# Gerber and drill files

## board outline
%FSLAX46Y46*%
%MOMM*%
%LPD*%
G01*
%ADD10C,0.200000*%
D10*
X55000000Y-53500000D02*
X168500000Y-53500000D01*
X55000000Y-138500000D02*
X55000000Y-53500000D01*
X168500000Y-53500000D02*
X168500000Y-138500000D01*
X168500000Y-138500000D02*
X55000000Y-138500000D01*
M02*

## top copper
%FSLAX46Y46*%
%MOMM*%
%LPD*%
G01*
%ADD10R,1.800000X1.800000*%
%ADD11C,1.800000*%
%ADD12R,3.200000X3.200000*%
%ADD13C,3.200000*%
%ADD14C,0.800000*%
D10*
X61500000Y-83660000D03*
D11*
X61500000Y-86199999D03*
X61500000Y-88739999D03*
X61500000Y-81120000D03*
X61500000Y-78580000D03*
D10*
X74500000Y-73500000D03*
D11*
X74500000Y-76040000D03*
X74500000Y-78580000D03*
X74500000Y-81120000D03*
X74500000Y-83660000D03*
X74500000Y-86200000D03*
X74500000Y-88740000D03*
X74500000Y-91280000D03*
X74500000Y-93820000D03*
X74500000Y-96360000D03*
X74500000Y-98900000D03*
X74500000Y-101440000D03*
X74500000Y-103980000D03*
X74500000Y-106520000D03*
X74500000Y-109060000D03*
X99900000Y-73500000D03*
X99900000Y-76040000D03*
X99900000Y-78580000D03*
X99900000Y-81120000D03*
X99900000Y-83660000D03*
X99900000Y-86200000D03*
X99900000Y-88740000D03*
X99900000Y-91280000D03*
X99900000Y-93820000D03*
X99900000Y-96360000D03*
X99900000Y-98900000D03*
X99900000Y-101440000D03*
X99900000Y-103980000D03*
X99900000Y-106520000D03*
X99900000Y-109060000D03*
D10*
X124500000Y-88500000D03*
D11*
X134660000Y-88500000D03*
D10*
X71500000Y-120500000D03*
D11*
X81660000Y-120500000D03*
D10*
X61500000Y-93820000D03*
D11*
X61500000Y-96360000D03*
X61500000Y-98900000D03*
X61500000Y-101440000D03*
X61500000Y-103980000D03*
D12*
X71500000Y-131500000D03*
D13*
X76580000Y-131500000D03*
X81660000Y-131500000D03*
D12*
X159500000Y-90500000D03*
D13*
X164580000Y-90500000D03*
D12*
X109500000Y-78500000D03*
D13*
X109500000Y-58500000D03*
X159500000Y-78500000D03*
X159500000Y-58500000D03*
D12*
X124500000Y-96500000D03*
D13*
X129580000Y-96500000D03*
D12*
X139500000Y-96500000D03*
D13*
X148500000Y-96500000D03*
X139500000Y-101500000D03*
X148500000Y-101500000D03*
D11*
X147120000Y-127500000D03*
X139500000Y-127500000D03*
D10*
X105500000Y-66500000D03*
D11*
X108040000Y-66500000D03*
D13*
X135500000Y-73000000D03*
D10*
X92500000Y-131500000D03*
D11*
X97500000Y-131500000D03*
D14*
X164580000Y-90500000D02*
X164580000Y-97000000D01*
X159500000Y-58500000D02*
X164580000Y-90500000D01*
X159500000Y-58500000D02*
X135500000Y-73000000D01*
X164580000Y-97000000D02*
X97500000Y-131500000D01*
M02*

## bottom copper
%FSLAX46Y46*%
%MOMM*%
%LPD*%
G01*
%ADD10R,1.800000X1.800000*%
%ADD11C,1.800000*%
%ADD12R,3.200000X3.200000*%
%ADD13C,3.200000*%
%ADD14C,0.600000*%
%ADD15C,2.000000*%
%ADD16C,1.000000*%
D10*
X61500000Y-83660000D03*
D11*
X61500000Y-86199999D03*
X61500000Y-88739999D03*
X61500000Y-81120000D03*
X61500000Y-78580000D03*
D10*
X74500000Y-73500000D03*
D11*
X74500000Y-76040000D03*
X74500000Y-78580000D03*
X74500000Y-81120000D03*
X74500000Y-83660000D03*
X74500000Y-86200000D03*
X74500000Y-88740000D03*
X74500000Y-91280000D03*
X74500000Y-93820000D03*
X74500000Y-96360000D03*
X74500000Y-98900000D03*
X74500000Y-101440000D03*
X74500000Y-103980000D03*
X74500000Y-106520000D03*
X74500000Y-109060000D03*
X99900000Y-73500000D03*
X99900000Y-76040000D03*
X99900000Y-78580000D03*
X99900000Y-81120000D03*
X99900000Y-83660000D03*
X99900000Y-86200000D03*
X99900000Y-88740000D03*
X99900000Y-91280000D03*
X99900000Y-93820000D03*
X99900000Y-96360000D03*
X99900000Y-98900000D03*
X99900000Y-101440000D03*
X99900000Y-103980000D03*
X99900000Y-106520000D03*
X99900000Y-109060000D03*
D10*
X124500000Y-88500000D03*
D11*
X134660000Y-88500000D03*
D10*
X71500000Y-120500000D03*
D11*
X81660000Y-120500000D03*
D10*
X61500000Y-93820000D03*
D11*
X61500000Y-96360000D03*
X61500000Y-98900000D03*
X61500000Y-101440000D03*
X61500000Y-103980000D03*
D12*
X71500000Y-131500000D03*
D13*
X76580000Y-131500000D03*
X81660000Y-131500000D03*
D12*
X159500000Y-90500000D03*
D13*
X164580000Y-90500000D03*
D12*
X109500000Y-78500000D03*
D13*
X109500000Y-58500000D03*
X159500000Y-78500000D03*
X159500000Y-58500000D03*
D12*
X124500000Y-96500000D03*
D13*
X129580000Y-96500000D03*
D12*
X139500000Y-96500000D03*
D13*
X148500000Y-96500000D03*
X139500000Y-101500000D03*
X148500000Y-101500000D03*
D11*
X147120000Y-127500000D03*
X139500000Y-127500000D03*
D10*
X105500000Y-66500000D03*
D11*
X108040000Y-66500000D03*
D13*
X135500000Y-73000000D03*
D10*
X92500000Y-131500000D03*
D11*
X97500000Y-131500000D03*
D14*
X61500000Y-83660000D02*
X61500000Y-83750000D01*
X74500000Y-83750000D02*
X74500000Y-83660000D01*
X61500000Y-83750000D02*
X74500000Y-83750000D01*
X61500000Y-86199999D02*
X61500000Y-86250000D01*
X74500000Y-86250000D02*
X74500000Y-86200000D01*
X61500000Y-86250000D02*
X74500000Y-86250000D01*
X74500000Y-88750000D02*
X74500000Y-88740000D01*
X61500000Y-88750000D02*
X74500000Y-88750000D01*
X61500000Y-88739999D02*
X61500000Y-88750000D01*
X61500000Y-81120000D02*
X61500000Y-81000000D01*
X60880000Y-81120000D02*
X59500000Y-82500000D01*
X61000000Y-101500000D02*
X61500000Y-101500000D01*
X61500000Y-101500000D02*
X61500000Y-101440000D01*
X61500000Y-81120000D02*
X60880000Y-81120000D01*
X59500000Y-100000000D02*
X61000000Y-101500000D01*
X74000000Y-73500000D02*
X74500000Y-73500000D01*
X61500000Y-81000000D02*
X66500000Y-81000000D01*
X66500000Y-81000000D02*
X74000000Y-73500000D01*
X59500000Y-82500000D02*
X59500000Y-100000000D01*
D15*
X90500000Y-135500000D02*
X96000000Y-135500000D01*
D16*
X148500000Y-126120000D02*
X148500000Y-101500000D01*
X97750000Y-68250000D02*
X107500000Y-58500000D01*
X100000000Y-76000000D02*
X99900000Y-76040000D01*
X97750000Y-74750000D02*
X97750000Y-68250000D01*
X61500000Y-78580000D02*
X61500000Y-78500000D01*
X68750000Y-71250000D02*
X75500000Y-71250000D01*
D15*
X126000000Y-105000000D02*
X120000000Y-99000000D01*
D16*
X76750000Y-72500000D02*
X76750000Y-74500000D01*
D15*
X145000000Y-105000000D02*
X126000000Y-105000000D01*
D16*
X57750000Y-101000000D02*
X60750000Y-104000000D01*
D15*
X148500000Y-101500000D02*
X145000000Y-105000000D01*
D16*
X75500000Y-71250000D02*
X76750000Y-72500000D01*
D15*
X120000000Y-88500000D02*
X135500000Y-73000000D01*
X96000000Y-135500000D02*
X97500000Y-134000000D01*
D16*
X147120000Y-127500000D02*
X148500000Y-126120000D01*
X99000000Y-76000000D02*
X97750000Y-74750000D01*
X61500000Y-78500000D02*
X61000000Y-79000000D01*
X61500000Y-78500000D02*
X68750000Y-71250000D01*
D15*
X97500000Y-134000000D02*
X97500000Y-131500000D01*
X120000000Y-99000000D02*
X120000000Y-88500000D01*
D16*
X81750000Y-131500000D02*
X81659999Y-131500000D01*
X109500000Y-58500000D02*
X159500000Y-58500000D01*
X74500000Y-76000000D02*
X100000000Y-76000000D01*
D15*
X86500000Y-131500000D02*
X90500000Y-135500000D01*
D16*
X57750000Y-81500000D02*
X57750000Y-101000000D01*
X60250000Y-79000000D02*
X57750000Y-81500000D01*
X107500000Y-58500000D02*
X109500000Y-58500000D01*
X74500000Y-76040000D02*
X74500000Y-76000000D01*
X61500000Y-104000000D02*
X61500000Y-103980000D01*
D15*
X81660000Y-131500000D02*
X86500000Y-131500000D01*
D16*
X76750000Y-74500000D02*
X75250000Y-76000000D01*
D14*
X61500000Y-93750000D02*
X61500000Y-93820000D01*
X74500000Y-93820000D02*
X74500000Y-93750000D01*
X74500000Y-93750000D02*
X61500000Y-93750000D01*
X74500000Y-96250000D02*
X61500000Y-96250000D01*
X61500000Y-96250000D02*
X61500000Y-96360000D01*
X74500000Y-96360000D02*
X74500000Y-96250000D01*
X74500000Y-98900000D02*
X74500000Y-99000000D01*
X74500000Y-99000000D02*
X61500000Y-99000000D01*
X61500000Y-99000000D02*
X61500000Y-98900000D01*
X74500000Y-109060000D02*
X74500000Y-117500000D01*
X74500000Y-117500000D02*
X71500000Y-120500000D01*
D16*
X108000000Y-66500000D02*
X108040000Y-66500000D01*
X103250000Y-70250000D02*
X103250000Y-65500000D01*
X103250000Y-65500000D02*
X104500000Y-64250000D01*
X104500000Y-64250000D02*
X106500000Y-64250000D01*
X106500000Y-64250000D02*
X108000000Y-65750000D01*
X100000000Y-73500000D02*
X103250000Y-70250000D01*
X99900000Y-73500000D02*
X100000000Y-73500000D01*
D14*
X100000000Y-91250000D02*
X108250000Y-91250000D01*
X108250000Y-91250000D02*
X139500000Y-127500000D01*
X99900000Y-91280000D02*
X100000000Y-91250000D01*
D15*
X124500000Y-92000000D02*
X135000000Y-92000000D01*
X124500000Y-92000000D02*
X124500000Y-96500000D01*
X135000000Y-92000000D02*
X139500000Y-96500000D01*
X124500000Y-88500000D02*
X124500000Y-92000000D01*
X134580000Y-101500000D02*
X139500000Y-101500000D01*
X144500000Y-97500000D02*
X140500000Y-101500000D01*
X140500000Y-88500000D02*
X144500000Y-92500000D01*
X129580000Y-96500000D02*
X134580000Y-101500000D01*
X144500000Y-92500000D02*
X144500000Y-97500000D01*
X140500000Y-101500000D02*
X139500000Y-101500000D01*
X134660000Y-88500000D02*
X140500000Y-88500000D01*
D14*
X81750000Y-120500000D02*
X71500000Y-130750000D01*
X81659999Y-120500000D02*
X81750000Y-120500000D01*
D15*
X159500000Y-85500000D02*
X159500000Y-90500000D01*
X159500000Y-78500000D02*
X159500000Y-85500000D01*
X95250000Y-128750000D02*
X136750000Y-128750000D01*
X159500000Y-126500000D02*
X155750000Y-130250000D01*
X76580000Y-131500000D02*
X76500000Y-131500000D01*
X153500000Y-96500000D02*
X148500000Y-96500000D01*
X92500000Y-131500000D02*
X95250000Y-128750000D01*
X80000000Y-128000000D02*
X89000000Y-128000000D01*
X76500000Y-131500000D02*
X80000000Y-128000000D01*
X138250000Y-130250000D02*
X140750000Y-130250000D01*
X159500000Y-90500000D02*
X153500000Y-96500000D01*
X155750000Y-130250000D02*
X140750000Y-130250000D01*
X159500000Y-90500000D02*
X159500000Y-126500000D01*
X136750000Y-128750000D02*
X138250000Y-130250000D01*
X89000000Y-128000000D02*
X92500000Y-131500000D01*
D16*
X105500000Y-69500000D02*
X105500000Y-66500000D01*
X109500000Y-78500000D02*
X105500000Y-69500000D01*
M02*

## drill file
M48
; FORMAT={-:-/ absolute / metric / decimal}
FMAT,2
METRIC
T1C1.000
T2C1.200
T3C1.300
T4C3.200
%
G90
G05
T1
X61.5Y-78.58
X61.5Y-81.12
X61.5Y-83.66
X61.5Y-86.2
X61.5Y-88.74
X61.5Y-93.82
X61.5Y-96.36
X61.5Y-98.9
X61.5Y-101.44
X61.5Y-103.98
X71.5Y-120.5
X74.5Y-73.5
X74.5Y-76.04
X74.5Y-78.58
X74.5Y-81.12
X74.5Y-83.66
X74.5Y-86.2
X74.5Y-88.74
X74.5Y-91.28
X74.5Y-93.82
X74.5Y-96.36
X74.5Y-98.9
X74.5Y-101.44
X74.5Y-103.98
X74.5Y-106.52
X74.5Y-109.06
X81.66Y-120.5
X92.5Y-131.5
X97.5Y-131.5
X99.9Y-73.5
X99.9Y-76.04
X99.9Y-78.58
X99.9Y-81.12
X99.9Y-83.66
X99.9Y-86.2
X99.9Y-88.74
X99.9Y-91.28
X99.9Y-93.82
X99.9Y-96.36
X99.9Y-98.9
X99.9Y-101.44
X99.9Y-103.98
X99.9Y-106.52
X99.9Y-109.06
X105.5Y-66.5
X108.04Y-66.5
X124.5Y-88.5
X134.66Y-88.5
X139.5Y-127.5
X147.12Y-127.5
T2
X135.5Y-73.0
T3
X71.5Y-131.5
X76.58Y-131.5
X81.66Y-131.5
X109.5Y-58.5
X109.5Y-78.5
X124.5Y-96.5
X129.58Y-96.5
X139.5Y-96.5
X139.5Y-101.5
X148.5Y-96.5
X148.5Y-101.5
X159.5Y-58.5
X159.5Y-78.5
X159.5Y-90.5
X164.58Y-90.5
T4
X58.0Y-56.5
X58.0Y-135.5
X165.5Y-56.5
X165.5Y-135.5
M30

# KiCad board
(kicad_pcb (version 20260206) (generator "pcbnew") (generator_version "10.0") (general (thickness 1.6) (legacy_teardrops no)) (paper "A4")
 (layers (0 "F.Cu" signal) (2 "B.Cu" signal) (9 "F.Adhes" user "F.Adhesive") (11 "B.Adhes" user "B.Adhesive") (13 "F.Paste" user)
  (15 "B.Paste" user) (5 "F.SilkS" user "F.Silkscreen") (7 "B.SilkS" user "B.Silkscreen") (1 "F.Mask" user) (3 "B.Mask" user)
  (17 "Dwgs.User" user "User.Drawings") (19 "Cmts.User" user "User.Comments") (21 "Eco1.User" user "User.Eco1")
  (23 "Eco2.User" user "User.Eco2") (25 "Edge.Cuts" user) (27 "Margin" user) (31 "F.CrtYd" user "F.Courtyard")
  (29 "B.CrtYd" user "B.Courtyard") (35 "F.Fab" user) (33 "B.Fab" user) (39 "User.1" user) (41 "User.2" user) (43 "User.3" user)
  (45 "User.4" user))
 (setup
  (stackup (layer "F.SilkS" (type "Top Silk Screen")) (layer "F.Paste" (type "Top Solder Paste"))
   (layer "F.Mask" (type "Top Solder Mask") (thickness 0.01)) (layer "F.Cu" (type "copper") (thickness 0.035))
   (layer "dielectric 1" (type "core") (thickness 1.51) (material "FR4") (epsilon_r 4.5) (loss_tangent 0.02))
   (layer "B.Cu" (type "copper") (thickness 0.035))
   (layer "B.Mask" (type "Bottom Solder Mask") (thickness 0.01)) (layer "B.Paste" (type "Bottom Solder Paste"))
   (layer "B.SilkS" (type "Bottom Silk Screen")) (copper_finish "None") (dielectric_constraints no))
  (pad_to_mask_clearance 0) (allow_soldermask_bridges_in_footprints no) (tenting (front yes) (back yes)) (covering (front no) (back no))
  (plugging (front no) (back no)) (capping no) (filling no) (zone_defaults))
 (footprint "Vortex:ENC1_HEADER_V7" (layer "F.Cu") (at 61.5 83.5 -90)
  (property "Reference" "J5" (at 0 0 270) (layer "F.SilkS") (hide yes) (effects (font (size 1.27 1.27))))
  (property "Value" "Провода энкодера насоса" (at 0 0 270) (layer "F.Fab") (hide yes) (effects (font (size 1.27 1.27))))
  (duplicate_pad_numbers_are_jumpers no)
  (pad "1" thru_hole rect (at 0.16 0 270) (size 1.8 1.8) (drill 1) (layers "*.Cu") (remove_unused_layers no) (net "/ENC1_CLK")
   (thermal_bridge_angle 45))
  (pad "2" thru_hole circle (at 2.699999 0 270) (size 1.8 1.8) (drill 1) (layers "*.Cu") (remove_unused_layers no) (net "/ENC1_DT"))
  (pad "3" thru_hole circle (at 5.239999 0 270) (size 1.8 1.8) (drill 1) (layers "*.Cu") (remove_unused_layers no) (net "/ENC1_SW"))
  (pad "4" thru_hole circle (at -2.38 0 270) (size 1.8 1.8) (drill 1) (layers "*.Cu") (remove_unused_layers no) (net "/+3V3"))
  (pad "5" thru_hole circle (at -4.92 0 270) (size 1.8 1.8) (drill 1) (layers "*.Cu") (remove_unused_layers no) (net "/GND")))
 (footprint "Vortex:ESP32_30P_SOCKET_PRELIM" (layer "F.Cu") (at 74.5 73.5)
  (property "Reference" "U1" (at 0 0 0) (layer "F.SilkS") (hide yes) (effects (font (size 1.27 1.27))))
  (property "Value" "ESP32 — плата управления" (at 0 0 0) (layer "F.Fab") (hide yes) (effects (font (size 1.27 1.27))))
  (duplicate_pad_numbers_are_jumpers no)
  (pad "1" thru_hole rect (at 0 0) (size 1.8 1.8) (drill 1) (layers "*.Cu") (remove_unused_layers no) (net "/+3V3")
   (thermal_bridge_angle 45))
  (pad "2" thru_hole circle (at 0 2.54) (size 1.8 1.8) (drill 1) (layers "*.Cu") (remove_unused_layers no) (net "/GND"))
  (pad "3" thru_hole circle (at 0 5.08) (size 1.8 1.8) (drill 1) (layers "*.Cu") (remove_unused_layers no) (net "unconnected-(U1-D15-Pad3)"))
  (pad "4" thru_hole circle (at 0 7.62) (size 1.8 1.8) (drill 1) (layers "*.Cu") (remove_unused_layers no) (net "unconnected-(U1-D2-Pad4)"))
  (pad "5" thru_hole circle (at 0 10.16) (size 1.8 1.8) (drill 1) (layers "*.Cu") (remove_unused_layers no) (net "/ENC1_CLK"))
  (pad "6" thru_hole circle (at 0 12.7) (size 1.8 1.8) (drill 1) (layers "*.Cu") (remove_unused_layers no) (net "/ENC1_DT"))
  (pad "7" thru_hole circle (at 0 15.24) (size 1.8 1.8) (drill 1) (layers "*.Cu") (remove_unused_layers no) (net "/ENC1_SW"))
  (pad "8" thru_hole circle (at 0 17.78) (size 1.8 1.8) (drill 1) (layers "*.Cu") (remove_unused_layers no) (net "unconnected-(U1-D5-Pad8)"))
  (pad "9" thru_hole circle (at 0 20.32) (size 1.8 1.8) (drill 1) (layers "*.Cu") (remove_unused_layers no) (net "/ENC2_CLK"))
  (pad "10" thru_hole circle (at 0 22.86) (size 1.8 1.8) (drill 1) (layers "*.Cu") (remove_unused_layers no) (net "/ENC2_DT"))
  (pad "11" thru_hole circle (at 0 25.4) (size 1.8 1.8) (drill 1) (layers "*.Cu") (remove_unused_layers no) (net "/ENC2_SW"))
  (pad "12" thru_hole circle (at 0 27.94) (size 1.8 1.8) (drill 1) (layers "*.Cu") (remove_unused_layers no)
   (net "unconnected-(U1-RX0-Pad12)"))
  (pad "13" thru_hole circle (at 0 30.48) (size 1.8 1.8) (drill 1) (layers "*.Cu") (remove_unused_layers no)
   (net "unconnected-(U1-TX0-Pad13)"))
  (pad "14" thru_hole circle (at 0 33.02) (size 1.8 1.8) (drill 1) (layers "*.Cu") (remove_unused_layers no)
   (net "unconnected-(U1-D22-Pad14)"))
  (pad "15" thru_hole circle (at 0 35.56) (size 1.8 1.8) (drill 1) (layers "*.Cu") (remove_unused_layers no) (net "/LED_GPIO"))
  (pad "16" thru_hole circle (at 25.4 0) (size 1.8 1.8) (drill 1) (layers "*.Cu") (remove_unused_layers no) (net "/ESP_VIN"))
  (pad "17" thru_hole circle (at 25.4 2.54) (size 1.8 1.8) (drill 1) (layers "*.Cu") (remove_unused_layers no) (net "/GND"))
  (pad "18" thru_hole circle (at 25.4 5.08) (size 1.8 1.8) (drill 1) (layers "*.Cu") (remove_unused_layers no)
   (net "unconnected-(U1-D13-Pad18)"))
  (pad "19" thru_hole circle (at 25.4 7.62) (size 1.8 1.8) (drill 1) (layers "*.Cu") (remove_unused_layers no)
   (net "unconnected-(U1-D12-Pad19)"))
  (pad "20" thru_hole circle (at 25.4 10.16) (size 1.8 1.8) (drill 1) (layers "*.Cu") (remove_unused_layers no)
   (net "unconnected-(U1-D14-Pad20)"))
  (pad "21" thru_hole circle (at 25.4 12.7) (size 1.8 1.8) (drill 1) (layers "*.Cu") (remove_unused_layers no)
   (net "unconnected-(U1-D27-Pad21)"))
  (pad "22" thru_hole circle (at 25.4 15.24) (size 1.8 1.8) (drill 1) (layers "*.Cu") (remove_unused_layers no)
   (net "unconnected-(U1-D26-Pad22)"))
  (pad "23" thru_hole circle (at 25.4 17.78) (size 1.8 1.8) (drill 1) (layers "*.Cu") (remove_unused_layers no) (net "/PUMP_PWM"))
  (pad "24" thru_hole circle (at 25.4 20.32) (size 1.8 1.8) (drill 1) (layers "*.Cu") (remove_unused_layers no)
   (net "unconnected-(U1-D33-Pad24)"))
  (pad "25" thru_hole circle (at 25.4 22.86) (size 1.8 1.8) (drill 1) (layers "*.Cu") (remove_unused_layers no)
   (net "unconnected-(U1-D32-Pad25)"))
  (pad "26" thru_hole circle (at 25.4 25.4) (size 1.8 1.8) (drill 1) (layers "*.Cu") (remove_unused_layers no)
   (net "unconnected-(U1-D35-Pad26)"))
  (pad "27" thru_hole circle (at 25.4 27.94) (size 1.8 1.8) (drill 1) (layers "*.Cu") (remove_unused_layers no)
   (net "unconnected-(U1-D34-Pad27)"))
  (pad "28" thru_hole circle (at 25.4 30.48) (size 1.8 1.8) (drill 1) (layers "*.Cu") (remove_unused_layers no)
   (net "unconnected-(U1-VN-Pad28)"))
  (pad "29" thru_hole circle (at 25.4 33.02) (size 1.8 1.8) (drill 1) (layers "*.Cu") (remove_unused_layers no)
   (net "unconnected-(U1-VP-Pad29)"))
  (pad "30" thru_hole circle (at 25.4 35.56) (size 1.8 1.8) (drill 1) (layers "*.Cu") (remove_unused_layers no)
   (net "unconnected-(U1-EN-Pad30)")))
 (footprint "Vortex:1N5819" (layer "F.Cu") (at 124.5 88.5)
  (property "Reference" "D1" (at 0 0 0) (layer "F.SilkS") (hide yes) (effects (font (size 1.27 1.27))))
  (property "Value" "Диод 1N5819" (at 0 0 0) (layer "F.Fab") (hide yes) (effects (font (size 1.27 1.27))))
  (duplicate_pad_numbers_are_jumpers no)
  (pad "1" thru_hole rect (at 0 0) (size 1.8 1.8) (drill 1) (layers "*.Cu") (remove_unused_layers no) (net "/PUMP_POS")
   (thermal_bridge_angle 45))
  (pad "2" thru_hole circle (at 10.16 0) (size 1.8 1.8) (drill 1) (layers "*.Cu") (remove_unused_layers no) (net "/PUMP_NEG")))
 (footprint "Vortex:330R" (layer "F.Cu") (at 71.5 120.5)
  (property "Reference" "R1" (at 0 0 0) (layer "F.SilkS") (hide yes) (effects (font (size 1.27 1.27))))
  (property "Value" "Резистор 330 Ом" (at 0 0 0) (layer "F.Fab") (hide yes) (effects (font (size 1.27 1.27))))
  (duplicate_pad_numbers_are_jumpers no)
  (pad "1" thru_hole rect (at 0 0) (size 1.8 1.8) (drill 1) (layers "*.Cu") (remove_unused_layers no) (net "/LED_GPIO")
   (thermal_bridge_angle 45))
  (pad "2" thru_hole circle (at 10.16 0) (size 1.8 1.8) (drill 1) (layers "*.Cu") (remove_unused_layers no) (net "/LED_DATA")))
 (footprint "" (layer "F.Cu") (at 58 135.5)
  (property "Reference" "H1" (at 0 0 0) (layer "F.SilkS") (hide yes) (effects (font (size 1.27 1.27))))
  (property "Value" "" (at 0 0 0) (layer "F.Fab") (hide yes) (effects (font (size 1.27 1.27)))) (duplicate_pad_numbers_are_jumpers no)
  (pad "" np_thru_hole circle (at 0 0) (size 3.2 3.2) (drill 3.2) (layers "*.Cu")))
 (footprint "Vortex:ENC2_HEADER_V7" (layer "F.Cu") (at 61.5 96.5 -90)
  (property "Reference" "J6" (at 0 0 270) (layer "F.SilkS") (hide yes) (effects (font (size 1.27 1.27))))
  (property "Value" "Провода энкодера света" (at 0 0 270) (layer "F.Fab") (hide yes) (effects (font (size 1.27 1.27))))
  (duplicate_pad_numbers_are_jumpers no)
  (pad "1" thru_hole rect (at -2.68 0 270) (size 1.8 1.8) (drill 1) (layers "*.Cu") (remove_unused_layers no) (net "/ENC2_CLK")
   (thermal_bridge_angle 45))
  (pad "2" thru_hole circle (at -0.14 0 270) (size 1.8 1.8) (drill 1) (layers "*.Cu") (remove_unused_layers no) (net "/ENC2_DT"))
  (pad "3" thru_hole circle (at 2.4 0 270) (size 1.8 1.8) (drill 1) (layers "*.Cu") (remove_unused_layers no) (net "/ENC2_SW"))
  (pad "4" thru_hole circle (at 4.94 0 270) (size 1.8 1.8) (drill 1) (layers "*.Cu") (remove_unused_layers no) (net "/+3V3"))
  (pad "5" thru_hole circle (at 7.48 0 270) (size 1.8 1.8) (drill 1) (layers "*.Cu") (remove_unused_layers no) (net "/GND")))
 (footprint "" (layer "F.Cu") (at 58 56.5)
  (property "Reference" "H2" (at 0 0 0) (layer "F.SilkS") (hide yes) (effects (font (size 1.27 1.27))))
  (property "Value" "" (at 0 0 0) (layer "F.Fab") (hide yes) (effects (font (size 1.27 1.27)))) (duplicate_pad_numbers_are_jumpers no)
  (pad "" np_thru_hole circle (at 0 0) (size 3.2 3.2) (drill 3.2) (layers "*.Cu")))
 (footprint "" (layer "F.Cu") (at 165.5 135.5)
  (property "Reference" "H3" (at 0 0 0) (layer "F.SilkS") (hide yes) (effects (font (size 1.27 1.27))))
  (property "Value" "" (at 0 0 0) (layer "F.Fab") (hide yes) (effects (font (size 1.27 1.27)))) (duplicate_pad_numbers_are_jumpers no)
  (pad "" np_thru_hole circle (at 0 0) (size 3.2 3.2) (drill 3.2) (layers "*.Cu")))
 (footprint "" (layer "F.Cu") (at 165.5 56.5)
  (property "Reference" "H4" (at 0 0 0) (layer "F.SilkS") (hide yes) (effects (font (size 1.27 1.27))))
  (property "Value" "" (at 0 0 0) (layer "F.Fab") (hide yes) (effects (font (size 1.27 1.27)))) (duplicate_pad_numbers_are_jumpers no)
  (pad "" np_thru_hole circle (at 0 0) (size 3.2 3.2) (drill 3.2) (layers "*.Cu")))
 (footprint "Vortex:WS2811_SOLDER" (layer "F.Cu") (at 71.5 131.5)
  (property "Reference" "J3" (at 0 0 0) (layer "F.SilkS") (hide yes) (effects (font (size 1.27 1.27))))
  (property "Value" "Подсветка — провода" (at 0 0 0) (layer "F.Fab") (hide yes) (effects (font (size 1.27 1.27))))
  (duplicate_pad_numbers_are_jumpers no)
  (pad "1" thru_hole rect (at 0 0) (size 3.2 3.2) (drill 1.3) (layers "*.Cu") (remove_unused_layers no) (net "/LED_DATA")
   (thermal_bridge_angle 45))
  (pad "2" thru_hole circle (at 5.08 0) (size 3.2 3.2) (drill 1.3) (layers "*.Cu") (remove_unused_layers no) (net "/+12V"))
  (pad "3" thru_hole circle (at 10.16 0) (size 3.2 3.2) (drill 1.3) (layers "*.Cu") (remove_unused_layers no) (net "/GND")))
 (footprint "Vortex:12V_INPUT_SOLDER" (layer "F.Cu") (at 159.5 90.5)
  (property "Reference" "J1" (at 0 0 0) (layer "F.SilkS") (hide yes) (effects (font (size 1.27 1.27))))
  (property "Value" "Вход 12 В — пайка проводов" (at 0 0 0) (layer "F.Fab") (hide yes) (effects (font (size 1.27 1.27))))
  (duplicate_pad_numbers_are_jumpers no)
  (pad "1" thru_hole rect (at 0 0) (size 3.2 3.2) (drill 1.3) (layers "*.Cu") (remove_unused_layers no) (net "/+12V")
   (thermal_bridge_angle 45))
  (pad "2" thru_hole circle (at 5.08 0) (size 3.2 3.2) (drill 1.3) (layers "*.Cu") (remove_unused_layers no) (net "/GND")))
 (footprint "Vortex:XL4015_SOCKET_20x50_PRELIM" (layer "F.Cu") (at 109.5 78.5 90)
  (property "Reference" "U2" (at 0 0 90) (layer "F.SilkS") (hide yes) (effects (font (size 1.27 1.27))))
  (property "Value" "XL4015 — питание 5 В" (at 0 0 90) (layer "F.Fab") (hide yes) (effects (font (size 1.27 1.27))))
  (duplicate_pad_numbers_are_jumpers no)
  (pad "1" thru_hole rect (at 0 0 90) (size 3.2 3.2) (drill 1.3) (layers "*.Cu") (remove_unused_layers no) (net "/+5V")
   (thermal_bridge_angle 45))
  (pad "2" thru_hole circle (at 20 0 90) (size 3.2 3.2) (drill 1.3) (layers "*.Cu") (remove_unused_layers no) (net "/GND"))
  (pad "3" thru_hole circle (at 0 50 90) (size 3.2 3.2) (drill 1.3) (layers "*.Cu") (remove_unused_layers no) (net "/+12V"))
  (pad "4" thru_hole circle (at 20 50 90) (size 3.2 3.2) (drill 1.3) (layers "*.Cu") (remove_unused_layers no) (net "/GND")))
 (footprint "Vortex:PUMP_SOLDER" (layer "F.Cu") (at 124.5 96.5)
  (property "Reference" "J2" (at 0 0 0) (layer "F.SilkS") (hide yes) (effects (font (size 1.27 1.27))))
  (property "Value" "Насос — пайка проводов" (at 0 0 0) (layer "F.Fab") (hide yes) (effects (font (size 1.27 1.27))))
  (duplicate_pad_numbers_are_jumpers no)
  (pad "1" thru_hole rect (at 0 0) (size 3.2 3.2) (drill 1.3) (layers "*.Cu") (remove_unused_layers no) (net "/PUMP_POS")
   (thermal_bridge_angle 45))
  (pad "2" thru_hole circle (at 5.08 0) (size 3.2 3.2) (drill 1.3) (layers "*.Cu") (remove_unused_layers no) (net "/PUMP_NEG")))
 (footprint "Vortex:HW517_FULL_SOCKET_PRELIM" (layer "F.Cu") (at 139.5 96.5)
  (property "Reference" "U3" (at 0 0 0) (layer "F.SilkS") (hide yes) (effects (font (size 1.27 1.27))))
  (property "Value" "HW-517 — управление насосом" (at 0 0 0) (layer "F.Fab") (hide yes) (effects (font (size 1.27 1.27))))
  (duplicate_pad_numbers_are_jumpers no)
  (pad "1" thru_hole rect (at 0 0) (size 3.2 3.2) (drill 1.3) (layers "*.Cu") (remove_unused_layers no) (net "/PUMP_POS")
   (thermal_bridge_angle 45))
  (pad "2" thru_hole circle (at 9 0) (size 3.2 3.2) (drill 1.3) (layers "*.Cu") (remove_unused_layers no) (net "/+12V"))
  (pad "3" thru_hole circle (at 0 5) (size 3.2 3.2) (drill 1.3) (layers "*.Cu") (remove_unused_layers no) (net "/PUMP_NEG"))
  (pad "4" thru_hole circle (at 9 5) (size 3.2 3.2) (drill 1.3) (layers "*.Cu") (remove_unused_layers no) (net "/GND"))
  (pad "5" thru_hole circle (at 7.62 31) (size 1.8 1.8) (drill 1) (layers "*.Cu") (remove_unused_layers no) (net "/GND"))
  (pad "6" thru_hole circle (at 0 31) (size 1.8 1.8) (drill 1) (layers "*.Cu") (remove_unused_layers no) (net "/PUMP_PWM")))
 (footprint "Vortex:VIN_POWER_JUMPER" (layer "F.Cu") (at 105.5 66.5)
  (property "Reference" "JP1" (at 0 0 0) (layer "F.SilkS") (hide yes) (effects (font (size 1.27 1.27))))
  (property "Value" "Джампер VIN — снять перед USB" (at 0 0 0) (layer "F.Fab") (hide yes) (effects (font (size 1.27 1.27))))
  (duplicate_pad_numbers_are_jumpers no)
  (pad "1" thru_hole rect (at 0 0) (size 1.8 1.8) (drill 1) (layers "*.Cu") (remove_unused_layers no) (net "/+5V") (thermal_bridge_angle 45))
  (pad "2" thru_hole circle (at 2.54 0) (size 1.8 1.8) (drill 1) (layers "*.Cu") (remove_unused_layers no) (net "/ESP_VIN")))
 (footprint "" (layer "F.Cu") (at 135.5 73)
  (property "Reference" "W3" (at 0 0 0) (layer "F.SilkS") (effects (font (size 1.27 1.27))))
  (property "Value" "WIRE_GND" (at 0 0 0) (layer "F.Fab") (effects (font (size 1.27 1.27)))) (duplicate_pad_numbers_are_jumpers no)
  (pad "1" thru_hole circle (at 0 0) (size 3.2 3.2) (drill 1.2) (layers "*.Cu") (remove_unused_layers no) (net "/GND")))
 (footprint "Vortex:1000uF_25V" (layer "F.Cu") (at 92.5 131.5)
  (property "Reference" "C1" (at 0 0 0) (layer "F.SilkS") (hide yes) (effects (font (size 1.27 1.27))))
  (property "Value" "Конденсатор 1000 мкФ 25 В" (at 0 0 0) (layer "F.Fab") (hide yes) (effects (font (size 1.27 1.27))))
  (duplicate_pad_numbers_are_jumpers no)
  (pad "1" thru_hole rect (at 0 0) (size 1.8 1.8) (drill 1) (layers "*.Cu") (remove_unused_layers no) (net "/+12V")
   (thermal_bridge_angle 45))
  (pad "2" thru_hole circle (at 5 0) (size 1.8 1.8) (drill 1) (layers "*.Cu") (remove_unused_layers no) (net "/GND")))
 (gr_line (start 55 53.5) (end 168.5 53.5) (stroke (width 0.2) (type default)) (layer "Edge.Cuts"))
 (gr_line (start 55 138.5) (end 55 53.5) (stroke (width 0.2) (type default)) (layer "Edge.Cuts"))
 (gr_line (start 168.5 53.5) (end 168.5 138.5) (stroke (width 0.2) (type default)) (layer "Edge.Cuts"))
 (gr_line (start 168.5 138.5) (end 55 138.5) (stroke (width 0.2) (type default)) (layer "Edge.Cuts"))
 (segment (start 61.5 83.66) (end 61.5 83.75) (width 0.6) (layer "B.Cu") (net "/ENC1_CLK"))
 (segment (start 74.5 83.75) (end 74.5 83.66) (width 0.6) (layer "B.Cu") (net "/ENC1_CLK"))
 (segment (start 61.5 83.75) (end 74.5 83.75) (width 0.6) (layer "B.Cu") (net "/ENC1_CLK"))
 (segment (start 61.5 86.199999) (end 61.5 86.25) (width 0.6) (layer "B.Cu") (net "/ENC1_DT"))
 (segment (start 74.5 86.25) (end 74.5 86.2) (width 0.6) (layer "B.Cu") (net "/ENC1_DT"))
 (segment (start 61.5 86.25) (end 74.5 86.25) (width 0.6) (layer "B.Cu") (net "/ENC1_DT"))
 (segment (start 74.5 88.75) (end 74.5 88.74) (width 0.6) (layer "B.Cu") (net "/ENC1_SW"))
 (segment (start 61.5 88.75) (end 74.5 88.75) (width 0.6) (layer "B.Cu") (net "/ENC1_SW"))
 (segment (start 61.5 88.739999) (end 61.5 88.75) (width 0.6) (layer "B.Cu") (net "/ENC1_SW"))
 (segment (start 61.5 81.12) (end 61.5 81) (width 0.6) (layer "B.Cu") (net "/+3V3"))
 (segment (start 60.88 81.12) (end 59.5 82.5) (width 0.6) (layer "B.Cu") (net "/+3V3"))
 (segment (start 61 101.5) (end 61.5 101.5) (width 0.6) (layer "B.Cu") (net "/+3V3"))
 (segment (start 61.5 101.5) (end 61.5 101.44) (width 0.6) (layer "B.Cu") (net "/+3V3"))
 (segment (start 61.5 81.12) (end 60.88 81.12) (width 0.6) (layer "B.Cu") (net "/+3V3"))
 (segment (start 59.5 100) (end 61 101.5) (width 0.6) (layer "B.Cu") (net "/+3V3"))
 (segment (start 74 73.5) (end 74.5 73.5) (width 0.6) (layer "B.Cu") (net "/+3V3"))
 (segment (start 61.5 81) (end 66.5 81) (width 0.6) (layer "B.Cu") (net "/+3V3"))
 (segment (start 66.5 81) (end 74 73.5) (width 0.6) (layer "B.Cu") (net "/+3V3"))
 (segment (start 59.5 82.5) (end 59.5 100) (width 0.6) (layer "B.Cu") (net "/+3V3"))
 (segment (start 164.58 90.5) (end 164.58 97) (width 0.8) (layer "F.Cu") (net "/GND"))
 (segment (start 159.5 58.5) (end 164.58 90.5) (width 0.8) (layer "F.Cu") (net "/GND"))
 (segment (start 159.5 58.5) (end 135.5 73) (width 0.8) (layer "F.Cu") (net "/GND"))
 (segment (start 164.58 97) (end 97.5 131.5) (width 0.8) (layer "F.Cu") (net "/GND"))
 (segment (start 90.5 135.5) (end 96 135.5) (width 2) (layer "B.Cu") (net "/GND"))
 (segment (start 148.5 126.12) (end 148.5 101.5) (width 1) (layer "B.Cu") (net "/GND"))
 (segment (start 97.75 68.25) (end 107.5 58.5) (width 1) (layer "B.Cu") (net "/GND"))
 (segment (start 100 76) (end 99.9 76.04) (width 1) (layer "B.Cu") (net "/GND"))
 (segment (start 97.75 74.75) (end 97.75 68.25) (width 1) (layer "B.Cu") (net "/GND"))
 (segment (start 61.5 78.58) (end 61.5 78.5) (width 1) (layer "B.Cu") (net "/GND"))
 (segment (start 68.75 71.25) (end 75.5 71.25) (width 1) (layer "B.Cu") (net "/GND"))
 (segment (start 126 105) (end 120 99) (width 2) (layer "B.Cu") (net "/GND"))
 (segment (start 76.75 72.5) (end 76.75 74.5) (width 1) (layer "B.Cu") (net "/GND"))
 (segment (start 145 105) (end 126 105) (width 2) (layer "B.Cu") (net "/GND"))
 (segment (start 57.75 101) (end 60.75 104) (width 1) (layer "B.Cu") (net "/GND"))
 (segment (start 148.5 101.5) (end 145 105) (width 2) (layer "B.Cu") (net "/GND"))
 (segment (start 75.5 71.25) (end 76.75 72.5) (width 1) (layer "B.Cu") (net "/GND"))
 (segment (start 120 88.5) (end 135.5 73) (width 2) (layer "B.Cu") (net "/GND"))
 (segment (start 96 135.5) (end 97.5 134) (width 2) (layer "B.Cu") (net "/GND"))
 (segment (start 147.12 127.5) (end 148.5 126.12) (width 1) (layer "B.Cu") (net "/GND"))
 (segment (start 99 76) (end 97.75 74.75) (width 1) (layer "B.Cu") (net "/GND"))
 (segment (start 61.5 78.5) (end 61 79) (width 1) (layer "B.Cu") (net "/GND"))
 (segment (start 61.5 78.5) (end 68.75 71.25) (width 1) (layer "B.Cu") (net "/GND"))
 (segment (start 97.5 134) (end 97.5 131.5) (width 2) (layer "B.Cu") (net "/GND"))
 (segment (start 120 99) (end 120 88.5) (width 2) (layer "B.Cu") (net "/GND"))
 (segment (start 81.75 131.5) (end 81.659999 131.5) (width 1) (layer "B.Cu") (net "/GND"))
 (segment (start 109.5 58.5) (end 159.5 58.5) (width 1) (layer "B.Cu") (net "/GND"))
 (segment (start 74.5 76) (end 100 76) (width 1) (layer "B.Cu") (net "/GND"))
 (segment (start 86.5 131.5) (end 90.5 135.5) (width 2) (layer "B.Cu") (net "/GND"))
 (segment (start 57.75 81.5) (end 57.75 101) (width 1) (layer "B.Cu") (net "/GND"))
 (segment (start 60.25 79) (end 57.75 81.5) (width 1) (layer "B.Cu") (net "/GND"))
 (segment (start 107.5 58.5) (end 109.5 58.5) (width 1) (layer "B.Cu") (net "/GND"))
 (segment (start 74.5 76.04) (end 74.5 76) (width 1) (layer "B.Cu") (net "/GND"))
 (segment (start 61.5 104) (end 61.5 103.98) (width 1) (layer "B.Cu") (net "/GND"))
 (segment (start 81.66 131.5) (end 86.5 131.5) (width 2) (layer "B.Cu") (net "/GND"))
 (segment (start 76.75 74.5) (end 75.25 76) (width 1) (layer "B.Cu") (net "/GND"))
 (segment (start 61.5 93.75) (end 61.5 93.82) (width 0.6) (layer "B.Cu") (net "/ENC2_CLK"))
 (segment (start 74.5 93.82) (end 74.5 93.75) (width 0.6) (layer "B.Cu") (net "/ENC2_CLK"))
 (segment (start 74.5 93.75) (end 61.5 93.75) (width 0.6) (layer "B.Cu") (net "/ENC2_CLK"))
 (segment (start 74.5 96.25) (end 61.5 96.25) (width 0.6) (layer "B.Cu") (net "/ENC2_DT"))
 (segment (start 61.5 96.25) (end 61.5 96.36) (width 0.6) (layer "B.Cu") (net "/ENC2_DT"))
 (segment (start 74.5 96.36) (end 74.5 96.25) (width 0.6) (layer "B.Cu") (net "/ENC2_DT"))
 (segment (start 74.5 98.9) (end 74.5 99) (width 0.6) (layer "B.Cu") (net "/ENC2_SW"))
 (segment (start 74.5 99) (end 61.5 99) (width 0.6) (layer "B.Cu") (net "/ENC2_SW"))
 (segment (start 61.5 99) (end 61.5 98.9) (width 0.6) (layer "B.Cu") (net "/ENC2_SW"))
 (segment (start 74.5 109.06) (end 74.5 117.5) (width 0.6) (layer "B.Cu") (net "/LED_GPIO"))
 (segment (start 74.5 117.5) (end 71.5 120.5) (width 0.6) (layer "B.Cu") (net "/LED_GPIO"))
 (segment (start 108 66.5) (end 108.04 66.5) (width 1) (layer "B.Cu") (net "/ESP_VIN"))
 (segment (start 103.25 70.25) (end 103.25 65.5) (width 1) (layer "B.Cu") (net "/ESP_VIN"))
 (segment (start 103.25 65.5) (end 104.5 64.25) (width 1) (layer "B.Cu") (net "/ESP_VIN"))
 (segment (start 104.5 64.25) (end 106.5 64.25) (width 1) (layer "B.Cu") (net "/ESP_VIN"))
 (segment (start 106.5 64.25) (end 108 65.75) (width 1) (layer "B.Cu") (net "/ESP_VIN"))
 (segment (start 100 73.5) (end 103.25 70.25) (width 1) (layer "B.Cu") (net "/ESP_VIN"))
 (segment (start 99.9 73.5) (end 100 73.5) (width 1) (layer "B.Cu") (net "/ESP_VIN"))
 (segment (start 100 91.25) (end 108.25 91.25) (width 0.6) (layer "B.Cu") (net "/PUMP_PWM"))
 (segment (start 108.25 91.25) (end 139.5 127.5) (width 0.6) (layer "B.Cu") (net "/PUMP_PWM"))
 (segment (start 99.9 91.28) (end 100 91.25) (width 0.6) (layer "B.Cu") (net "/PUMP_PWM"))
 (segment (start 124.5 92) (end 135 92) (width 2) (layer "B.Cu") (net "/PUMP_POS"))
 (segment (start 124.5 92) (end 124.5 96.5) (width 2) (layer "B.Cu") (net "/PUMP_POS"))
 (segment (start 135 92) (end 139.5 96.5) (width 2) (layer "B.Cu") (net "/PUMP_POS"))
 (segment (start 124.5 88.5) (end 124.5 92) (width 2) (layer "B.Cu") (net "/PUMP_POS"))
 (segment (start 134.58 101.5) (end 139.5 101.5) (width 2) (layer "B.Cu") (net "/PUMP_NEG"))
 (segment (start 144.5 97.5) (end 140.5 101.5) (width 2) (layer "B.Cu") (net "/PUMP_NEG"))
 (segment (start 140.5 88.5) (end 144.5 92.5) (width 2) (layer "B.Cu") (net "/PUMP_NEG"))
 (segment (start 129.58 96.5) (end 134.58 101.5) (width 2) (layer "B.Cu") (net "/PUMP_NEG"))
 (segment (start 144.5 92.5) (end 144.5 97.5) (width 2) (layer "B.Cu") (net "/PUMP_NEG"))
 (segment (start 140.5 101.5) (end 139.5 101.5) (width 2) (layer "B.Cu") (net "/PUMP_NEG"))
 (segment (start 134.66 88.5) (end 140.5 88.5) (width 2) (layer "B.Cu") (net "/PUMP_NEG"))
 (segment (start 81.75 120.5) (end 71.5 130.75) (width 0.6) (layer "B.Cu") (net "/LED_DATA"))
 (segment (start 81.659999 120.5) (end 81.75 120.5) (width 0.6) (layer "B.Cu") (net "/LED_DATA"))
 (segment (start 159.5 85.5) (end 159.5 90.5) (width 2) (layer "B.Cu") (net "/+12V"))
 (segment (start 159.5 78.5) (end 159.5 85.5) (width 2) (layer "B.Cu") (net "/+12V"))
 (segment (start 95.25 128.75) (end 136.75 128.75) (width 2) (layer "B.Cu") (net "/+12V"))
 (segment (start 159.5 126.5) (end 155.75 130.25) (width 2) (layer "B.Cu") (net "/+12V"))
 (segment (start 76.58 131.5) (end 76.5 131.5) (width 2) (layer "B.Cu") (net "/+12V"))
 (segment (start 153.5 96.5) (end 148.5 96.5) (width 2) (layer "B.Cu") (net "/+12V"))
 (segment (start 92.5 131.5) (end 95.25 128.75) (width 2) (layer "B.Cu") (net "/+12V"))
 (segment (start 80 128) (end 89 128) (width 2) (layer "B.Cu") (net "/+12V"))
 (segment (start 76.5 131.5) (end 80 128) (width 2) (layer "B.Cu") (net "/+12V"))
 (segment (start 138.25 130.25) (end 140.75 130.25) (width 2) (layer "B.Cu") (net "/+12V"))
 (segment (start 159.5 90.5) (end 153.5 96.5) (width 2) (layer "B.Cu") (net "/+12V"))
 (segment (start 155.75 130.25) (end 140.75 130.25) (width 2) (layer "B.Cu") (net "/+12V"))
 (segment (start 159.5 90.5) (end 159.5 126.5) (width 2) (layer "B.Cu") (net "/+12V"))
 (segment (start 136.75 128.75) (end 138.25 130.25) (width 2) (layer "B.Cu") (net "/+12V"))
 (segment (start 89 128) (end 92.5 131.5) (width 2) (layer "B.Cu") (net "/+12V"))
 (segment (start 105.5 69.5) (end 105.5 66.5) (width 1) (layer "B.Cu") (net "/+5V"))
 (segment (start 109.5 78.5) (end 105.5 69.5) (width 1) (layer "B.Cu") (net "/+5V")))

